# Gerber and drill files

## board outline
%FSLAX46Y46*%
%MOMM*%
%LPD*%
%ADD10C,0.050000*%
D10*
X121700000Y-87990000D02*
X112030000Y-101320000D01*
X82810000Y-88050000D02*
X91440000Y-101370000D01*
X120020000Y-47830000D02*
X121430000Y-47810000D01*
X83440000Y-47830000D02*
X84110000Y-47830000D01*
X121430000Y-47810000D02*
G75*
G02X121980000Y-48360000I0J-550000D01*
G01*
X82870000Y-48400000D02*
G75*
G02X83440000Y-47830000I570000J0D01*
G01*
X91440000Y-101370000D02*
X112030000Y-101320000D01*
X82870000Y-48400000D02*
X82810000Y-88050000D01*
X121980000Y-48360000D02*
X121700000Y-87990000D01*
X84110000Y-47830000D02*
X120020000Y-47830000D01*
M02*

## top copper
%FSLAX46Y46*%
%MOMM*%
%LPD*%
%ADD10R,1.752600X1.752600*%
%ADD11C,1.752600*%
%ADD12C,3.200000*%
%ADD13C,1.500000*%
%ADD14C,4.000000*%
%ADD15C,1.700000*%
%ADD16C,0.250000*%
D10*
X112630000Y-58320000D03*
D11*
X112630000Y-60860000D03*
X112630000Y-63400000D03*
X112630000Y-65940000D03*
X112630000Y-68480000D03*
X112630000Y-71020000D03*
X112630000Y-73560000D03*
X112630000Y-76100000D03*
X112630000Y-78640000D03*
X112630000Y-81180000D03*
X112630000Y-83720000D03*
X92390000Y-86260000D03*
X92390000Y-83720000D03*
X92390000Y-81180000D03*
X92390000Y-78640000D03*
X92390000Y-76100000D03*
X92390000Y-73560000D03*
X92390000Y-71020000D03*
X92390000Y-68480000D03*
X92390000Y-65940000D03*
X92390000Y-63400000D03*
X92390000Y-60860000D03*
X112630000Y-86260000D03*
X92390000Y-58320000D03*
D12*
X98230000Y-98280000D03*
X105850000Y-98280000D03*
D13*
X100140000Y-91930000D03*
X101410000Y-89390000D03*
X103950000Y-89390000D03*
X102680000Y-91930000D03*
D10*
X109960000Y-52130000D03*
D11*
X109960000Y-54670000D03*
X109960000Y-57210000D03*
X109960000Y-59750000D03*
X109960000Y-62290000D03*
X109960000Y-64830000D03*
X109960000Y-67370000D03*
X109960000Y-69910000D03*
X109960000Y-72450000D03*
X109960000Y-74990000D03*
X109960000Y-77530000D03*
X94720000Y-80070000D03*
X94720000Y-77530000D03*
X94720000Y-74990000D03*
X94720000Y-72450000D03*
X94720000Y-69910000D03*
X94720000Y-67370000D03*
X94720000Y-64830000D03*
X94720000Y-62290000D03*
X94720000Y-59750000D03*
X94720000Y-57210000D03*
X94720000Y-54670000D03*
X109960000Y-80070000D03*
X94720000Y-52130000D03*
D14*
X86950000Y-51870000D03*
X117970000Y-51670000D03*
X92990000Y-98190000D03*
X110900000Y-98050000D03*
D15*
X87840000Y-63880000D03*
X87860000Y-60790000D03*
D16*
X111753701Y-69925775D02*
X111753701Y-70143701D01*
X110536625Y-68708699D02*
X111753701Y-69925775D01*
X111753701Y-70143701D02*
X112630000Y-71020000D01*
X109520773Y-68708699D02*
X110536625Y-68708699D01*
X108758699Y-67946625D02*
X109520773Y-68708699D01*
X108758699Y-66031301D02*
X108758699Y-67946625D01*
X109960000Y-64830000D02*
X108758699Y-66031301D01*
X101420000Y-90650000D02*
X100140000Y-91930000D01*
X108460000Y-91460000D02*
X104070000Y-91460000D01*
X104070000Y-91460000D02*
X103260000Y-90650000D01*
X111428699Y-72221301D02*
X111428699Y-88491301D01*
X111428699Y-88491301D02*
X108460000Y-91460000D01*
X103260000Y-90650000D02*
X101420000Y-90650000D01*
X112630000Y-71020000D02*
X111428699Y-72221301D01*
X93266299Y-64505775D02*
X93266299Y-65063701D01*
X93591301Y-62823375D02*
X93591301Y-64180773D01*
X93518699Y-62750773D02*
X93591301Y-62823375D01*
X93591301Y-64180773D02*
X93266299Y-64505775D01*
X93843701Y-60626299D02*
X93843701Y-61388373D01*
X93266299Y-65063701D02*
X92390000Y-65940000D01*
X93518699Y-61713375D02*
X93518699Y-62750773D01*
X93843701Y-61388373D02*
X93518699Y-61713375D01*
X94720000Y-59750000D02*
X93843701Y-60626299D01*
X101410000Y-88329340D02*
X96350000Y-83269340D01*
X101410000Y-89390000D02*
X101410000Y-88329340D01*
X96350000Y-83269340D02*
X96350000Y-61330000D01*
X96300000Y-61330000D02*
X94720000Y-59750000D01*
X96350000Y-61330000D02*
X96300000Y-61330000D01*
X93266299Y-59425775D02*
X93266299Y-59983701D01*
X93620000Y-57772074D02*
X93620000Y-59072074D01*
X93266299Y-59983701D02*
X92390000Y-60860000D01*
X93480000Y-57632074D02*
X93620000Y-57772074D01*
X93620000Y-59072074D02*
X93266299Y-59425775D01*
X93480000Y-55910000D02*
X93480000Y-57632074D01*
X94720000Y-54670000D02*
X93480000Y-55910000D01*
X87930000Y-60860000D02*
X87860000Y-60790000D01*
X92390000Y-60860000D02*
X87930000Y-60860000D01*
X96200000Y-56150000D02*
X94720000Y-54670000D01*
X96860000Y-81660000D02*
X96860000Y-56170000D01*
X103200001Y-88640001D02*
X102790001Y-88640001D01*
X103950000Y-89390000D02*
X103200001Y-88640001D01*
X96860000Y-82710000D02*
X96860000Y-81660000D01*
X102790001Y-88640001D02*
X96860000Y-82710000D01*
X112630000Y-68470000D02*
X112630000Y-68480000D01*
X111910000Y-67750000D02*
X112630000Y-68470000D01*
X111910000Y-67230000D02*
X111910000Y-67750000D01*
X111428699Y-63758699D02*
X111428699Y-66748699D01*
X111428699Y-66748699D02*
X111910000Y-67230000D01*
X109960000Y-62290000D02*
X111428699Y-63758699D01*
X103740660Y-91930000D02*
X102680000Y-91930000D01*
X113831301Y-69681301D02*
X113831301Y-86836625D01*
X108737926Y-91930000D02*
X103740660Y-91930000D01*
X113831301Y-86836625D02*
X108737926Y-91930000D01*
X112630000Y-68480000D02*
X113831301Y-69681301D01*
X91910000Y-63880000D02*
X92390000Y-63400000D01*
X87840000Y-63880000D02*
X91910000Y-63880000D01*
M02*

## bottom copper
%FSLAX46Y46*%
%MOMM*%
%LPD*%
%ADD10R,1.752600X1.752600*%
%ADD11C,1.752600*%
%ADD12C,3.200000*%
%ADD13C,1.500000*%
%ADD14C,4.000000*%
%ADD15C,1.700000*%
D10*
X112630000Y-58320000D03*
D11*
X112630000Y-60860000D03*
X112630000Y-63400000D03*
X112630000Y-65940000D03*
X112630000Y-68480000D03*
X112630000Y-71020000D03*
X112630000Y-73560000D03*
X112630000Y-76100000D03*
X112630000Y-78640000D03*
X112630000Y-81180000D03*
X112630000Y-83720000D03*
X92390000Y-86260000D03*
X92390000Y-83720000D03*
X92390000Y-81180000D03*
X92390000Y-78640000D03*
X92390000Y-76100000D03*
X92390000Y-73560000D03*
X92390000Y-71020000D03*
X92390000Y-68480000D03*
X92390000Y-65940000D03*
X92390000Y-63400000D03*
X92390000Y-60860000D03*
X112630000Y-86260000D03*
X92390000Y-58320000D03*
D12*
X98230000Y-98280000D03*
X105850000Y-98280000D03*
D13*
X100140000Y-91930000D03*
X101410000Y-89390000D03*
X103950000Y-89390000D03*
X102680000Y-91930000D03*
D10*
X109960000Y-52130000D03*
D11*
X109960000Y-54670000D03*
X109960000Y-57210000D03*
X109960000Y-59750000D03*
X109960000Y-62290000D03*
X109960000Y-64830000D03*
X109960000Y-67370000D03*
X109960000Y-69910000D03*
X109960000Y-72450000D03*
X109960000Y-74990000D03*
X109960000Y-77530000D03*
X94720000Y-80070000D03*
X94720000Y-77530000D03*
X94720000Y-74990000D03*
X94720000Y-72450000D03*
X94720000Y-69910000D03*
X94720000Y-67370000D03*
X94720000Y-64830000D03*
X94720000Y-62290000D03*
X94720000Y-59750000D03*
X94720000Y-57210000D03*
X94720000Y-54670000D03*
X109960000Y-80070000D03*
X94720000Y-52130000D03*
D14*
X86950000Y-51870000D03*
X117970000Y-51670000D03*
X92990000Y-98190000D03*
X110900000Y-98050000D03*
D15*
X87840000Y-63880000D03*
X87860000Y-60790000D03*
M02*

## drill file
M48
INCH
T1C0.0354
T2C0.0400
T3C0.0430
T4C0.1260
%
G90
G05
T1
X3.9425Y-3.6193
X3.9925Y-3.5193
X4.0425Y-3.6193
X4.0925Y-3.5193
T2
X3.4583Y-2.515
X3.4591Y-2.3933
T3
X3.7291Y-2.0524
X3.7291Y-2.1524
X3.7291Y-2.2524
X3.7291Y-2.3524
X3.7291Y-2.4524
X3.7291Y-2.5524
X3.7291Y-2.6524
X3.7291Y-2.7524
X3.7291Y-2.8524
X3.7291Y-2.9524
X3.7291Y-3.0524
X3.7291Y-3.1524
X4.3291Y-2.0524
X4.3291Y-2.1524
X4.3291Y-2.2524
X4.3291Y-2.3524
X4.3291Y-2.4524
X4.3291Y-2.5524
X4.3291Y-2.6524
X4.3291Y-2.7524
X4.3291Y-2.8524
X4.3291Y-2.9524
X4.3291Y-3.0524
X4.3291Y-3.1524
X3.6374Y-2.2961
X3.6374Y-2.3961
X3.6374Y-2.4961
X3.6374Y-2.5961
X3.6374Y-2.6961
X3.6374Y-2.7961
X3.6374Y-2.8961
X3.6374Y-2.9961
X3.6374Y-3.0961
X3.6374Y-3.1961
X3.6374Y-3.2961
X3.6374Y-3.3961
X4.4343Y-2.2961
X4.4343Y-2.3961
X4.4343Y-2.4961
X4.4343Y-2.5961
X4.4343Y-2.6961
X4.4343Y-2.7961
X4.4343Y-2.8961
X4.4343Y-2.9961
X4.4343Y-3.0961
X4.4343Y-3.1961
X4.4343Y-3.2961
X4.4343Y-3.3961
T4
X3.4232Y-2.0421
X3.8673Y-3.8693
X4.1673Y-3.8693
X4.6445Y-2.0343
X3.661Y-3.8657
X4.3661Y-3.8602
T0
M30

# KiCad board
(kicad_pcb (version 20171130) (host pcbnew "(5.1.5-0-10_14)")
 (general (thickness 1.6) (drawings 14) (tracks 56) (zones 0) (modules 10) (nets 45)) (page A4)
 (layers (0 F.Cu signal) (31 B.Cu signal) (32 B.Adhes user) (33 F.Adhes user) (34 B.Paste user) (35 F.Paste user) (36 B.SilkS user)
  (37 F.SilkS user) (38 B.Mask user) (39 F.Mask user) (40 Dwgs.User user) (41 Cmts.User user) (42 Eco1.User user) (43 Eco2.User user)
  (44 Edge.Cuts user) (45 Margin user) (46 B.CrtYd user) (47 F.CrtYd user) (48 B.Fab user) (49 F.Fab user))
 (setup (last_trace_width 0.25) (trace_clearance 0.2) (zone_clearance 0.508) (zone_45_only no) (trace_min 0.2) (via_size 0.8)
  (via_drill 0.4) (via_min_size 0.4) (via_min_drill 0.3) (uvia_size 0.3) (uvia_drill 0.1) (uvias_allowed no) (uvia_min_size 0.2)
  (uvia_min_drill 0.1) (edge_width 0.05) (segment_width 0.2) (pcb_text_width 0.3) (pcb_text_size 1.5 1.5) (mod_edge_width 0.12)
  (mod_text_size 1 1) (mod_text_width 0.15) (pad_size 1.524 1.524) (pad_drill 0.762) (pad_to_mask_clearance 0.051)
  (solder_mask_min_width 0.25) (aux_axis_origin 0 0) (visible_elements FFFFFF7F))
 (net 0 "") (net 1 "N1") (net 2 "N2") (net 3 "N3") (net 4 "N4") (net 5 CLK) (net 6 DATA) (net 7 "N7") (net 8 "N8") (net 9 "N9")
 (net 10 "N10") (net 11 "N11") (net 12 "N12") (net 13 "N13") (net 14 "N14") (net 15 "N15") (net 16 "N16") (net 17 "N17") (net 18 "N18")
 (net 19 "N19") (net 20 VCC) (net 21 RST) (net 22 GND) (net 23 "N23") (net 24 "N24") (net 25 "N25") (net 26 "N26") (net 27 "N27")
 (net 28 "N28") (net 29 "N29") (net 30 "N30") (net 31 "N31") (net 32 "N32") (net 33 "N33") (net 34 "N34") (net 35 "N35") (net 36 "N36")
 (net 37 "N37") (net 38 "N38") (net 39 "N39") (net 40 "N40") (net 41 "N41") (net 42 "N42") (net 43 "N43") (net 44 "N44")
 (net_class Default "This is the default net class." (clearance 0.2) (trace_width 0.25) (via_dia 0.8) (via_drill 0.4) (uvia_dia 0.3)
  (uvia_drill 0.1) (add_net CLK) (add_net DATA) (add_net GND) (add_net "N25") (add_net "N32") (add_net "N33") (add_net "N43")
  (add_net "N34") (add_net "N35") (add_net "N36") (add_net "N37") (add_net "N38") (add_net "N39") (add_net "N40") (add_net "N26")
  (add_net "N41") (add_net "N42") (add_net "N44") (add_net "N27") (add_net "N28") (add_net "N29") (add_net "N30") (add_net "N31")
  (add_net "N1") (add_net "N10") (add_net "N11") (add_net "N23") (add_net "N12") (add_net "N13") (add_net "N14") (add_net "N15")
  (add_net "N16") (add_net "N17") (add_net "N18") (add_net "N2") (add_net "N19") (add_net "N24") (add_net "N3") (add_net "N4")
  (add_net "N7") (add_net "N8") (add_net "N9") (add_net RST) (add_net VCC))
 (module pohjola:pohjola (layer B.Cu) (at 102.27 67.5 180)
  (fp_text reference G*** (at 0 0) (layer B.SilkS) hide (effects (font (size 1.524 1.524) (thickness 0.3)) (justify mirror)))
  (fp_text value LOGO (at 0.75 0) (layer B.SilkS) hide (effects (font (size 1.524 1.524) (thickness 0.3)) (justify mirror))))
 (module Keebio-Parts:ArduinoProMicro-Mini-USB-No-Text (layer B.Cu) (at 102.51 72.29 270)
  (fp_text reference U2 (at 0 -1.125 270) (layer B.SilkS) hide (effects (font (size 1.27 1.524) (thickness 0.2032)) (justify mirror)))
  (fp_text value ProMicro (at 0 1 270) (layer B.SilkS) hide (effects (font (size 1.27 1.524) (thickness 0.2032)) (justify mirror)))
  (pad 1 thru_hole rect (at -13.97 -10.12 270) (size 1.7526 1.7526) (drill 1.0922) (layers *.Cu *.SilkS *.Mask) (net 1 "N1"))
  (pad 2 thru_hole circle (at -11.43 -10.12 270) (size 1.7526 1.7526) (drill 1.0922) (layers *.Cu *.SilkS *.Mask) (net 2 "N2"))
  (pad 3 thru_hole circle (at -8.89 -10.12 270) (size 1.7526 1.7526) (drill 1.0922) (layers *.Cu *.SilkS *.Mask) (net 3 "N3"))
  (pad 4 thru_hole circle (at -6.35 -10.12 270) (size 1.7526 1.7526) (drill 1.0922) (layers *.Cu *.SilkS *.Mask) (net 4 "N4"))
  (pad 5 thru_hole circle (at -3.81 -10.12 270) (size 1.7526 1.7526) (drill 1.0922) (layers *.Cu *.SilkS *.Mask) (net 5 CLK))
  (pad 6 thru_hole circle (at -1.27 -10.12 270) (size 1.7526 1.7526) (drill 1.0922) (layers *.Cu *.SilkS *.Mask) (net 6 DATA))
  (pad 7 thru_hole circle (at 1.27 -10.12 270) (size 1.7526 1.7526) (drill 1.0922) (layers *.Cu *.SilkS *.Mask) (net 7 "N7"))
  (pad 8 thru_hole circle (at 3.81 -10.12 270) (size 1.7526 1.7526) (drill 1.0922) (layers *.Cu *.SilkS *.Mask) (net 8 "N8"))
  (pad 9 thru_hole circle (at 6.35 -10.12 270) (size 1.7526 1.7526) (drill 1.0922) (layers *.Cu *.SilkS *.Mask) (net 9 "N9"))
  (pad 10 thru_hole circle (at 8.89 -10.12 270) (size 1.7526 1.7526) (drill 1.0922) (layers *.Cu *.SilkS *.Mask) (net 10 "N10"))
  (pad 11 thru_hole circle (at 11.43 -10.12 270) (size 1.7526 1.7526) (drill 1.0922) (layers *.Cu *.SilkS *.Mask) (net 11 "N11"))
  (pad 13 thru_hole circle (at 13.97 10.12 270) (size 1.7526 1.7526) (drill 1.0922) (layers *.Cu *.SilkS *.Mask) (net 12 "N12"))
  (pad 14 thru_hole circle (at 11.43 10.12 270) (size 1.7526 1.7526) (drill 1.0922) (layers *.Cu *.SilkS *.Mask) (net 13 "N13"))
  (pad 15 thru_hole circle (at 8.89 10.12 270) (size 1.7526 1.7526) (drill 1.0922) (layers *.Cu *.SilkS *.Mask) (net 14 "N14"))
  (pad 16 thru_hole circle (at 6.35 10.12 270) (size 1.7526 1.7526) (drill 1.0922) (layers *.Cu *.SilkS *.Mask) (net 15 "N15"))
  (pad 17 thru_hole circle (at 3.81 10.12 270) (size 1.7526 1.7526) (drill 1.0922) (layers *.Cu *.SilkS *.Mask) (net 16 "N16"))
  (pad 18 thru_hole circle (at 1.27 10.12 270) (size 1.7526 1.7526) (drill 1.0922) (layers *.Cu *.SilkS *.Mask) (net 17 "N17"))
  (pad 19 thru_hole circle (at -1.27 10.12 270) (size 1.7526 1.7526) (drill 1.0922) (layers *.Cu *.SilkS *.Mask) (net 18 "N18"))
  (pad 20 thru_hole circle (at -3.81 10.12 270) (size 1.7526 1.7526) (drill 1.0922) (layers *.Cu *.SilkS *.Mask) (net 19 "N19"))
  (pad 21 thru_hole circle (at -6.35 10.12 270) (size 1.7526 1.7526) (drill 1.0922) (layers *.Cu *.SilkS *.Mask) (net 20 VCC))
  (pad 22 thru_hole circle (at -8.89 10.12 270) (size 1.7526 1.7526) (drill 1.0922) (layers *.Cu *.SilkS *.Mask) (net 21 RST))
  (pad 23 thru_hole circle (at -11.43 10.12 270) (size 1.7526 1.7526) (drill 1.0922) (layers *.Cu *.SilkS *.Mask) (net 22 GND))
  (pad 12 thru_hole circle (at 13.97 -10.12 270) (size 1.7526 1.7526) (drill 1.0922) (layers *.Cu *.SilkS *.Mask) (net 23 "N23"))
  (pad 24 thru_hole circle (at -13.97 10.12 270) (size 1.7526 1.7526) (drill 1.0922) (layers *.Cu *.SilkS *.Mask) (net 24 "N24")))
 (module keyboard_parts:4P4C (layer F.Cu) (at 102.04 98.28)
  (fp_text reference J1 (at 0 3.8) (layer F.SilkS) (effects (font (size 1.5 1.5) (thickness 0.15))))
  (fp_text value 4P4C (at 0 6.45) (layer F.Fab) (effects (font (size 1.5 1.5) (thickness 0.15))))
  (pad 5 thru_hole circle (at -3.81 0) (size 3.2 3.2) (drill 3.2) (layers *.Cu *.Mask F.SilkS))
  (pad 6 thru_hole circle (at 3.81 0) (size 3.2 3.2) (drill 3.2) (layers *.Cu *.Mask F.SilkS))
  (pad 1 thru_hole circle (at -1.9 -6.35) (size 1.5 1.5) (drill 0.9) (layers *.Cu *.Mask F.SilkS) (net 6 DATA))
  (pad 2 thru_hole circle (at -0.63 -8.89) (size 1.5 1.5) (drill 0.9) (layers *.Cu *.Mask F.SilkS) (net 20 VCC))
  (pad 4 thru_hole circle (at 1.91 -8.89) (size 1.5 1.5) (drill 0.9) (layers *.Cu *.Mask F.SilkS) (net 22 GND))
  (pad 3 thru_hole circle (at 0.64 -6.35) (size 1.5 1.5) (drill 0.9) (layers *.Cu *.Mask F.SilkS) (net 5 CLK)))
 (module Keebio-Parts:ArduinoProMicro (layer B.Cu) (at 102.34 66.1 270)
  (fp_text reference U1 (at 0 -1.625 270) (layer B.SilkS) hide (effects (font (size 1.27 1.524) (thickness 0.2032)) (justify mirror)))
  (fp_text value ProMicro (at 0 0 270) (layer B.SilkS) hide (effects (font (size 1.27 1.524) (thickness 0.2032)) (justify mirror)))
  (pad 1 thru_hole rect (at -13.97 -7.62 270) (size 1.7526 1.7526) (drill 1.0922) (layers *.Cu *.SilkS *.Mask) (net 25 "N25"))
  (pad 2 thru_hole circle (at -11.43 -7.62 270) (size 1.7526 1.7526) (drill 1.0922) (layers *.Cu *.SilkS *.Mask) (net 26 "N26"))
  (pad 3 thru_hole circle (at -8.89 -7.62 270) (size 1.7526 1.7526) (drill 1.0922) (layers *.Cu *.SilkS *.Mask) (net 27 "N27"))
  (pad 4 thru_hole circle (at -6.35 -7.62 270) (size 1.7526 1.7526) (drill 1.0922) (layers *.Cu *.SilkS *.Mask) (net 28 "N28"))
  (pad 5 thru_hole circle (at -3.81 -7.62 270) (size 1.7526 1.7526) (drill 1.0922) (layers *.Cu *.SilkS *.Mask) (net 5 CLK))
  (pad 6 thru_hole circle (at -1.27 -7.62 270) (size 1.7526 1.7526) (drill 1.0922) (layers *.Cu *.SilkS *.Mask) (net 6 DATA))
  (pad 7 thru_hole circle (at 1.27 -7.62 270) (size 1.7526 1.7526) (drill 1.0922) (layers *.Cu *.SilkS *.Mask) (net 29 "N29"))
  (pad 8 thru_hole circle (at 3.81 -7.62 270) (size 1.7526 1.7526) (drill 1.0922) (layers *.Cu *.SilkS *.Mask) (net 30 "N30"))
  (pad 9 thru_hole circle (at 6.35 -7.62 270) (size 1.7526 1.7526) (drill 1.0922) (layers *.Cu *.SilkS *.Mask) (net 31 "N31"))
  (pad 10 thru_hole circle (at 8.89 -7.62 270) (size 1.7526 1.7526) (drill 1.0922) (layers *.Cu *.SilkS *.Mask) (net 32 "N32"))
  (pad 11 thru_hole circle (at 11.43 -7.62 270) (size 1.7526 1.7526) (drill 1.0922) (layers *.Cu *.SilkS *.Mask) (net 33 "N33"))
  (pad 13 thru_hole circle (at 13.97 7.62 270) (size 1.7526 1.7526) (drill 1.0922) (layers *.Cu *.SilkS *.Mask) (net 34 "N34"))
  (pad 14 thru_hole circle (at 11.43 7.62 270) (size 1.7526 1.7526) (drill 1.0922) (layers *.Cu *.SilkS *.Mask) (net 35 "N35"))
  (pad 15 thru_hole circle (at 8.89 7.62 270) (size 1.7526 1.7526) (drill 1.0922) (layers *.Cu *.SilkS *.Mask) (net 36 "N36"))
  (pad 16 thru_hole circle (at 6.35 7.62 270) (size 1.7526 1.7526) (drill 1.0922) (layers *.Cu *.SilkS *.Mask) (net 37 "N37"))
  (pad 17 thru_hole circle (at 3.81 7.62 270) (size 1.7526 1.7526) (drill 1.0922) (layers *.Cu *.SilkS *.Mask) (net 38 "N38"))
  (pad 18 thru_hole circle (at 1.27 7.62 270) (size 1.7526 1.7526) (drill 1.0922) (layers *.Cu *.SilkS *.Mask) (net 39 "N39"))
  (pad 19 thru_hole circle (at -1.27 7.62 270) (size 1.7526 1.7526) (drill 1.0922) (layers *.Cu *.SilkS *.Mask) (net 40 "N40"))
  (pad 20 thru_hole circle (at -3.81 7.62 270) (size 1.7526 1.7526) (drill 1.0922) (layers *.Cu *.SilkS *.Mask) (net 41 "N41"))
  (pad 21 thru_hole circle (at -6.35 7.62 270) (size 1.7526 1.7526) (drill 1.0922) (layers *.Cu *.SilkS *.Mask) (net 20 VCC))
  (pad 22 thru_hole circle (at -8.89 7.62 270) (size 1.7526 1.7526) (drill 1.0922) (layers *.Cu *.SilkS *.Mask) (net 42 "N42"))
  (pad 23 thru_hole circle (at -11.43 7.62 270) (size 1.7526 1.7526) (drill 1.0922) (layers *.Cu *.SilkS *.Mask) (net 22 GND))
  (pad 12 thru_hole circle (at 13.97 -7.62 270) (size 1.7526 1.7526) (drill 1.0922) (layers *.Cu *.SilkS *.Mask) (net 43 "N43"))
  (pad 24 thru_hole circle (at -13.97 7.62 270) (size 1.7526 1.7526) (drill 1.0922) (layers *.Cu *.SilkS *.Mask) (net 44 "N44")))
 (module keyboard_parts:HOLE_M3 (layer F.Cu) (at 86.95 51.87)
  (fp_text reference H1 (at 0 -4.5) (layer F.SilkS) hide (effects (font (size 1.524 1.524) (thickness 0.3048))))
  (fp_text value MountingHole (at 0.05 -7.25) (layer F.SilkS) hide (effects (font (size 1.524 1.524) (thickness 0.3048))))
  (pad 1 thru_hole circle (at 0 0) (size 4 4) (drill 3.2) (layers *.Cu *.Mask F.SilkS)))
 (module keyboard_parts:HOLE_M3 (layer F.Cu) (at 117.97 51.67)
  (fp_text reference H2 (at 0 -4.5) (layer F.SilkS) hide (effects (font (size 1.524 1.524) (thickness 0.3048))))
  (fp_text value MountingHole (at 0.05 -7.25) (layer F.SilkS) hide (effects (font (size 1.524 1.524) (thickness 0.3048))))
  (pad 1 thru_hole circle (at 0 0) (size 4 4) (drill 3.2) (layers *.Cu *.Mask F.SilkS)))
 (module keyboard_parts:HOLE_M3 (layer F.Cu) (at 92.99 98.19)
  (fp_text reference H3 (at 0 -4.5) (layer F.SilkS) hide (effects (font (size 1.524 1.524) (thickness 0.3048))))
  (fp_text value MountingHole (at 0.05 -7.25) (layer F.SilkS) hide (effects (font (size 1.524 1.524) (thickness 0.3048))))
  (pad 1 thru_hole circle (at 0 0) (size 4 4) (drill 3.2) (layers *.Cu *.Mask F.SilkS)))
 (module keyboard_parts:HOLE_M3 (layer F.Cu) (at 110.9 98.05)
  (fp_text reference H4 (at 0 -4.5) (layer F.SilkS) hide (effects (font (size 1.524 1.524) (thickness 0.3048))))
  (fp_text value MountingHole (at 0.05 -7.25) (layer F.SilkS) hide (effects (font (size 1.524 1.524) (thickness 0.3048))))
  (pad 1 thru_hole circle (at 0 0) (size 4 4) (drill 3.2) (layers *.Cu *.Mask F.SilkS)))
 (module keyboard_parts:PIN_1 (layer F.Cu) (at 87.84 63.88)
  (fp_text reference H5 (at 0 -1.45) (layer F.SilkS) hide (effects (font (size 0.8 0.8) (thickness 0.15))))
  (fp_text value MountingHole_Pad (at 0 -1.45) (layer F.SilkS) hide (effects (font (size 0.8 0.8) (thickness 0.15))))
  (pad 1 thru_hole circle (at 0 0) (size 1.7 1.7) (drill 1.016) (layers *.Cu *.Mask F.SilkS) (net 21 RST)))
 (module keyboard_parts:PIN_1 (layer F.Cu) (at 87.86 60.79)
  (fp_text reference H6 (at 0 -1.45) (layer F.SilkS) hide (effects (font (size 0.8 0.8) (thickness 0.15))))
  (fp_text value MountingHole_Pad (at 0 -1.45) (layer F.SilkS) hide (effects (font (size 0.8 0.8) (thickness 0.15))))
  (pad 1 thru_hole circle (at 0 0) (size 1.7 1.7) (drill 1.016) (layers *.Cu *.Mask F.SilkS) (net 22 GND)))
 (gr_line (start 121.7 87.99) (end 112.03 101.32) (layer Edge.Cuts) (width 0.05))
 (gr_line (start 82.81 88.05) (end 91.44 101.37) (layer Edge.Cuts) (width 0.05))
 (gr_line (start 120.02 47.83) (end 121.43 47.81) (layer Edge.Cuts) (width 0.05))
 (gr_line (start 83.44 47.83) (end 84.11 47.83) (layer Edge.Cuts) (width 0.05))
 (gr_arc (start 121.43 48.36) (end 121.98 48.36) (angle -90) (layer Edge.Cuts) (width 0.05))
 (gr_arc (start 83.44 48.4) (end 83.44 47.83) (angle -90) (layer Edge.Cuts) (width 0.05))
 (gr_line (start 91.44 101.37) (end 112.03 101.32) (layer Edge.Cuts) (width 0.05))
 (gr_line (start 82.87 48.4) (end 82.81 88.05) (layer Edge.Cuts) (width 0.05))
 (gr_line (start 121.98 48.36) (end 121.7 87.99) (layer Edge.Cuts) (width 0.05))
 (gr_line (start 84.11 47.83) (end 120.02 47.83) (layer Edge.Cuts) (width 0.05))
 (segment (start 111.753701 69.925775) (end 111.753701 70.143701) (width 0.25) (layer F.Cu) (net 6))
 (segment (start 110.536625 68.708699) (end 111.753701 69.925775) (width 0.25) (layer F.Cu) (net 6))
 (segment (start 111.753701 70.143701) (end 112.63 71.02) (width 0.25) (layer F.Cu) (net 6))
 (segment (start 109.520773 68.708699) (end 110.536625 68.708699) (width 0.25) (layer F.Cu) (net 6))
 (segment (start 108.758699 67.946625) (end 109.520773 68.708699) (width 0.25) (layer F.Cu) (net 6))
 (segment (start 108.758699 66.031301) (end 108.758699 67.946625) (width 0.25) (layer F.Cu) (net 6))
 (segment (start 109.96 64.83) (end 108.758699 66.031301) (width 0.25) (layer F.Cu) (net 6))
 (segment (start 101.42 90.65) (end 100.14 91.93) (width 0.25) (layer F.Cu) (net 6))
 (segment (start 108.46 91.46) (end 104.07 91.46) (width 0.25) (layer F.Cu) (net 6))
 (segment (start 104.07 91.46) (end 103.26 90.65) (width 0.25) (layer F.Cu) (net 6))
 (segment (start 111.428699 72.221301) (end 111.428699 88.491301) (width 0.25) (layer F.Cu) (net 6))
 (segment (start 111.428699 88.491301) (end 108.46 91.46) (width 0.25) (layer F.Cu) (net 6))
 (segment (start 103.26 90.65) (end 101.42 90.65) (width 0.25) (layer F.Cu) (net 6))
 (segment (start 112.63 71.02) (end 111.428699 72.221301) (width 0.25) (layer F.Cu) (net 6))
 (segment (start 93.266299 64.505775) (end 93.266299 65.063701) (width 0.25) (layer F.Cu) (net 20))
 (segment (start 93.591301 62.823375) (end 93.591301 64.180773) (width 0.25) (layer F.Cu) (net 20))
 (segment (start 93.518699 62.750773) (end 93.591301 62.823375) (width 0.25) (layer F.Cu) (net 20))
 (segment (start 93.591301 64.180773) (end 93.266299 64.505775) (width 0.25) (layer F.Cu) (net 20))
 (segment (start 93.843701 60.626299) (end 93.843701 61.388373) (width 0.25) (layer F.Cu) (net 20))
 (segment (start 93.266299 65.063701) (end 92.39 65.94) (width 0.25) (layer F.Cu) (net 20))
 (segment (start 93.518699 61.713375) (end 93.518699 62.750773) (width 0.25) (layer F.Cu) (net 20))
 (segment (start 93.843701 61.388373) (end 93.518699 61.713375) (width 0.25) (layer F.Cu) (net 20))
 (segment (start 94.72 59.75) (end 93.843701 60.626299) (width 0.25) (layer F.Cu) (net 20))
 (segment (start 101.41 88.32934) (end 96.35 83.26934) (width 0.25) (layer F.Cu) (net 20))
 (segment (start 101.41 89.39) (end 101.41 88.32934) (width 0.25) (layer F.Cu) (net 20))
 (segment (start 96.35 83.26934) (end 96.35 61.33) (width 0.25) (layer F.Cu) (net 20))
 (segment (start 96.3 61.33) (end 94.72 59.75) (width 0.25) (layer F.Cu) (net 20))
 (segment (start 96.35 61.33) (end 96.3 61.33) (width 0.25) (layer F.Cu) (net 20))
 (segment (start 93.266299 59.425775) (end 93.266299 59.983701) (width 0.25) (layer F.Cu) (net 22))
 (segment (start 93.62 57.772074) (end 93.62 59.072074) (width 0.25) (layer F.Cu) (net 22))
 (segment (start 93.266299 59.983701) (end 92.39 60.86) (width 0.25) (layer F.Cu) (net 22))
 (segment (start 93.48 57.632074) (end 93.62 57.772074) (width 0.25) (layer F.Cu) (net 22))
 (segment (start 93.62 59.072074) (end 93.266299 59.425775) (width 0.25) (layer F.Cu) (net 22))
 (segment (start 93.48 55.91) (end 93.48 57.632074) (width 0.25) (layer F.Cu) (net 22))
 (segment (start 94.72 54.67) (end 93.48 55.91) (width 0.25) (layer F.Cu) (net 22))
 (segment (start 87.93 60.86) (end 87.86 60.79) (width 0.25) (layer F.Cu) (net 22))
 (segment (start 92.39 60.86) (end 87.93 60.86) (width 0.25) (layer F.Cu) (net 22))
 (segment (start 96.2 56.15) (end 94.72 54.67) (width 0.25) (layer F.Cu) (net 22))
 (segment (start 96.86 81.66) (end 96.86 56.17) (width 0.25) (layer F.Cu) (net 22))
 (segment (start 103.200001 88.640001) (end 102.790001 88.640001) (width 0.25) (layer F.Cu) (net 22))
 (segment (start 103.95 89.39) (end 103.200001 88.640001) (width 0.25) (layer F.Cu) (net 22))
 (segment (start 96.86 82.71) (end 96.86 81.66) (width 0.25) (layer F.Cu) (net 22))
 (segment (start 102.790001 88.640001) (end 96.86 82.71) (width 0.25) (layer F.Cu) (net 22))
 (segment (start 112.63 68.47) (end 112.63 68.48) (width 0.25) (layer F.Cu) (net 5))
 (segment (start 111.91 67.75) (end 112.63 68.47) (width 0.25) (layer F.Cu) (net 5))
 (segment (start 111.91 67.23) (end 111.91 67.75) (width 0.25) (layer F.Cu) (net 5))
 (segment (start 111.428699 63.758699) (end 111.428699 66.748699) (width 0.25) (layer F.Cu) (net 5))
 (segment (start 111.428699 66.748699) (end 111.91 67.23) (width 0.25) (layer F.Cu) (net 5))
 (segment (start 109.96 62.29) (end 111.428699 63.758699) (width 0.25) (layer F.Cu) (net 5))
 (segment (start 103.74066 91.93) (end 102.68 91.93) (width 0.25) (layer F.Cu) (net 5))
 (segment (start 113.831301 69.681301) (end 113.831301 86.836625) (width 0.25) (layer F.Cu) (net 5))
 (segment (start 108.737926 91.93) (end 103.74066 91.93) (width 0.25) (layer F.Cu) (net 5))
 (segment (start 113.831301 86.836625) (end 108.737926 91.93) (width 0.25) (layer F.Cu) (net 5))
 (segment (start 112.63 68.48) (end 113.831301 69.681301) (width 0.25) (layer F.Cu) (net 5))
 (segment (start 91.91 63.88) (end 92.39 63.4) (width 0.25) (layer F.Cu) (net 21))
 (segment (start 87.84 63.88) (end 91.91 63.88) (width 0.25) (layer F.Cu) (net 21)))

